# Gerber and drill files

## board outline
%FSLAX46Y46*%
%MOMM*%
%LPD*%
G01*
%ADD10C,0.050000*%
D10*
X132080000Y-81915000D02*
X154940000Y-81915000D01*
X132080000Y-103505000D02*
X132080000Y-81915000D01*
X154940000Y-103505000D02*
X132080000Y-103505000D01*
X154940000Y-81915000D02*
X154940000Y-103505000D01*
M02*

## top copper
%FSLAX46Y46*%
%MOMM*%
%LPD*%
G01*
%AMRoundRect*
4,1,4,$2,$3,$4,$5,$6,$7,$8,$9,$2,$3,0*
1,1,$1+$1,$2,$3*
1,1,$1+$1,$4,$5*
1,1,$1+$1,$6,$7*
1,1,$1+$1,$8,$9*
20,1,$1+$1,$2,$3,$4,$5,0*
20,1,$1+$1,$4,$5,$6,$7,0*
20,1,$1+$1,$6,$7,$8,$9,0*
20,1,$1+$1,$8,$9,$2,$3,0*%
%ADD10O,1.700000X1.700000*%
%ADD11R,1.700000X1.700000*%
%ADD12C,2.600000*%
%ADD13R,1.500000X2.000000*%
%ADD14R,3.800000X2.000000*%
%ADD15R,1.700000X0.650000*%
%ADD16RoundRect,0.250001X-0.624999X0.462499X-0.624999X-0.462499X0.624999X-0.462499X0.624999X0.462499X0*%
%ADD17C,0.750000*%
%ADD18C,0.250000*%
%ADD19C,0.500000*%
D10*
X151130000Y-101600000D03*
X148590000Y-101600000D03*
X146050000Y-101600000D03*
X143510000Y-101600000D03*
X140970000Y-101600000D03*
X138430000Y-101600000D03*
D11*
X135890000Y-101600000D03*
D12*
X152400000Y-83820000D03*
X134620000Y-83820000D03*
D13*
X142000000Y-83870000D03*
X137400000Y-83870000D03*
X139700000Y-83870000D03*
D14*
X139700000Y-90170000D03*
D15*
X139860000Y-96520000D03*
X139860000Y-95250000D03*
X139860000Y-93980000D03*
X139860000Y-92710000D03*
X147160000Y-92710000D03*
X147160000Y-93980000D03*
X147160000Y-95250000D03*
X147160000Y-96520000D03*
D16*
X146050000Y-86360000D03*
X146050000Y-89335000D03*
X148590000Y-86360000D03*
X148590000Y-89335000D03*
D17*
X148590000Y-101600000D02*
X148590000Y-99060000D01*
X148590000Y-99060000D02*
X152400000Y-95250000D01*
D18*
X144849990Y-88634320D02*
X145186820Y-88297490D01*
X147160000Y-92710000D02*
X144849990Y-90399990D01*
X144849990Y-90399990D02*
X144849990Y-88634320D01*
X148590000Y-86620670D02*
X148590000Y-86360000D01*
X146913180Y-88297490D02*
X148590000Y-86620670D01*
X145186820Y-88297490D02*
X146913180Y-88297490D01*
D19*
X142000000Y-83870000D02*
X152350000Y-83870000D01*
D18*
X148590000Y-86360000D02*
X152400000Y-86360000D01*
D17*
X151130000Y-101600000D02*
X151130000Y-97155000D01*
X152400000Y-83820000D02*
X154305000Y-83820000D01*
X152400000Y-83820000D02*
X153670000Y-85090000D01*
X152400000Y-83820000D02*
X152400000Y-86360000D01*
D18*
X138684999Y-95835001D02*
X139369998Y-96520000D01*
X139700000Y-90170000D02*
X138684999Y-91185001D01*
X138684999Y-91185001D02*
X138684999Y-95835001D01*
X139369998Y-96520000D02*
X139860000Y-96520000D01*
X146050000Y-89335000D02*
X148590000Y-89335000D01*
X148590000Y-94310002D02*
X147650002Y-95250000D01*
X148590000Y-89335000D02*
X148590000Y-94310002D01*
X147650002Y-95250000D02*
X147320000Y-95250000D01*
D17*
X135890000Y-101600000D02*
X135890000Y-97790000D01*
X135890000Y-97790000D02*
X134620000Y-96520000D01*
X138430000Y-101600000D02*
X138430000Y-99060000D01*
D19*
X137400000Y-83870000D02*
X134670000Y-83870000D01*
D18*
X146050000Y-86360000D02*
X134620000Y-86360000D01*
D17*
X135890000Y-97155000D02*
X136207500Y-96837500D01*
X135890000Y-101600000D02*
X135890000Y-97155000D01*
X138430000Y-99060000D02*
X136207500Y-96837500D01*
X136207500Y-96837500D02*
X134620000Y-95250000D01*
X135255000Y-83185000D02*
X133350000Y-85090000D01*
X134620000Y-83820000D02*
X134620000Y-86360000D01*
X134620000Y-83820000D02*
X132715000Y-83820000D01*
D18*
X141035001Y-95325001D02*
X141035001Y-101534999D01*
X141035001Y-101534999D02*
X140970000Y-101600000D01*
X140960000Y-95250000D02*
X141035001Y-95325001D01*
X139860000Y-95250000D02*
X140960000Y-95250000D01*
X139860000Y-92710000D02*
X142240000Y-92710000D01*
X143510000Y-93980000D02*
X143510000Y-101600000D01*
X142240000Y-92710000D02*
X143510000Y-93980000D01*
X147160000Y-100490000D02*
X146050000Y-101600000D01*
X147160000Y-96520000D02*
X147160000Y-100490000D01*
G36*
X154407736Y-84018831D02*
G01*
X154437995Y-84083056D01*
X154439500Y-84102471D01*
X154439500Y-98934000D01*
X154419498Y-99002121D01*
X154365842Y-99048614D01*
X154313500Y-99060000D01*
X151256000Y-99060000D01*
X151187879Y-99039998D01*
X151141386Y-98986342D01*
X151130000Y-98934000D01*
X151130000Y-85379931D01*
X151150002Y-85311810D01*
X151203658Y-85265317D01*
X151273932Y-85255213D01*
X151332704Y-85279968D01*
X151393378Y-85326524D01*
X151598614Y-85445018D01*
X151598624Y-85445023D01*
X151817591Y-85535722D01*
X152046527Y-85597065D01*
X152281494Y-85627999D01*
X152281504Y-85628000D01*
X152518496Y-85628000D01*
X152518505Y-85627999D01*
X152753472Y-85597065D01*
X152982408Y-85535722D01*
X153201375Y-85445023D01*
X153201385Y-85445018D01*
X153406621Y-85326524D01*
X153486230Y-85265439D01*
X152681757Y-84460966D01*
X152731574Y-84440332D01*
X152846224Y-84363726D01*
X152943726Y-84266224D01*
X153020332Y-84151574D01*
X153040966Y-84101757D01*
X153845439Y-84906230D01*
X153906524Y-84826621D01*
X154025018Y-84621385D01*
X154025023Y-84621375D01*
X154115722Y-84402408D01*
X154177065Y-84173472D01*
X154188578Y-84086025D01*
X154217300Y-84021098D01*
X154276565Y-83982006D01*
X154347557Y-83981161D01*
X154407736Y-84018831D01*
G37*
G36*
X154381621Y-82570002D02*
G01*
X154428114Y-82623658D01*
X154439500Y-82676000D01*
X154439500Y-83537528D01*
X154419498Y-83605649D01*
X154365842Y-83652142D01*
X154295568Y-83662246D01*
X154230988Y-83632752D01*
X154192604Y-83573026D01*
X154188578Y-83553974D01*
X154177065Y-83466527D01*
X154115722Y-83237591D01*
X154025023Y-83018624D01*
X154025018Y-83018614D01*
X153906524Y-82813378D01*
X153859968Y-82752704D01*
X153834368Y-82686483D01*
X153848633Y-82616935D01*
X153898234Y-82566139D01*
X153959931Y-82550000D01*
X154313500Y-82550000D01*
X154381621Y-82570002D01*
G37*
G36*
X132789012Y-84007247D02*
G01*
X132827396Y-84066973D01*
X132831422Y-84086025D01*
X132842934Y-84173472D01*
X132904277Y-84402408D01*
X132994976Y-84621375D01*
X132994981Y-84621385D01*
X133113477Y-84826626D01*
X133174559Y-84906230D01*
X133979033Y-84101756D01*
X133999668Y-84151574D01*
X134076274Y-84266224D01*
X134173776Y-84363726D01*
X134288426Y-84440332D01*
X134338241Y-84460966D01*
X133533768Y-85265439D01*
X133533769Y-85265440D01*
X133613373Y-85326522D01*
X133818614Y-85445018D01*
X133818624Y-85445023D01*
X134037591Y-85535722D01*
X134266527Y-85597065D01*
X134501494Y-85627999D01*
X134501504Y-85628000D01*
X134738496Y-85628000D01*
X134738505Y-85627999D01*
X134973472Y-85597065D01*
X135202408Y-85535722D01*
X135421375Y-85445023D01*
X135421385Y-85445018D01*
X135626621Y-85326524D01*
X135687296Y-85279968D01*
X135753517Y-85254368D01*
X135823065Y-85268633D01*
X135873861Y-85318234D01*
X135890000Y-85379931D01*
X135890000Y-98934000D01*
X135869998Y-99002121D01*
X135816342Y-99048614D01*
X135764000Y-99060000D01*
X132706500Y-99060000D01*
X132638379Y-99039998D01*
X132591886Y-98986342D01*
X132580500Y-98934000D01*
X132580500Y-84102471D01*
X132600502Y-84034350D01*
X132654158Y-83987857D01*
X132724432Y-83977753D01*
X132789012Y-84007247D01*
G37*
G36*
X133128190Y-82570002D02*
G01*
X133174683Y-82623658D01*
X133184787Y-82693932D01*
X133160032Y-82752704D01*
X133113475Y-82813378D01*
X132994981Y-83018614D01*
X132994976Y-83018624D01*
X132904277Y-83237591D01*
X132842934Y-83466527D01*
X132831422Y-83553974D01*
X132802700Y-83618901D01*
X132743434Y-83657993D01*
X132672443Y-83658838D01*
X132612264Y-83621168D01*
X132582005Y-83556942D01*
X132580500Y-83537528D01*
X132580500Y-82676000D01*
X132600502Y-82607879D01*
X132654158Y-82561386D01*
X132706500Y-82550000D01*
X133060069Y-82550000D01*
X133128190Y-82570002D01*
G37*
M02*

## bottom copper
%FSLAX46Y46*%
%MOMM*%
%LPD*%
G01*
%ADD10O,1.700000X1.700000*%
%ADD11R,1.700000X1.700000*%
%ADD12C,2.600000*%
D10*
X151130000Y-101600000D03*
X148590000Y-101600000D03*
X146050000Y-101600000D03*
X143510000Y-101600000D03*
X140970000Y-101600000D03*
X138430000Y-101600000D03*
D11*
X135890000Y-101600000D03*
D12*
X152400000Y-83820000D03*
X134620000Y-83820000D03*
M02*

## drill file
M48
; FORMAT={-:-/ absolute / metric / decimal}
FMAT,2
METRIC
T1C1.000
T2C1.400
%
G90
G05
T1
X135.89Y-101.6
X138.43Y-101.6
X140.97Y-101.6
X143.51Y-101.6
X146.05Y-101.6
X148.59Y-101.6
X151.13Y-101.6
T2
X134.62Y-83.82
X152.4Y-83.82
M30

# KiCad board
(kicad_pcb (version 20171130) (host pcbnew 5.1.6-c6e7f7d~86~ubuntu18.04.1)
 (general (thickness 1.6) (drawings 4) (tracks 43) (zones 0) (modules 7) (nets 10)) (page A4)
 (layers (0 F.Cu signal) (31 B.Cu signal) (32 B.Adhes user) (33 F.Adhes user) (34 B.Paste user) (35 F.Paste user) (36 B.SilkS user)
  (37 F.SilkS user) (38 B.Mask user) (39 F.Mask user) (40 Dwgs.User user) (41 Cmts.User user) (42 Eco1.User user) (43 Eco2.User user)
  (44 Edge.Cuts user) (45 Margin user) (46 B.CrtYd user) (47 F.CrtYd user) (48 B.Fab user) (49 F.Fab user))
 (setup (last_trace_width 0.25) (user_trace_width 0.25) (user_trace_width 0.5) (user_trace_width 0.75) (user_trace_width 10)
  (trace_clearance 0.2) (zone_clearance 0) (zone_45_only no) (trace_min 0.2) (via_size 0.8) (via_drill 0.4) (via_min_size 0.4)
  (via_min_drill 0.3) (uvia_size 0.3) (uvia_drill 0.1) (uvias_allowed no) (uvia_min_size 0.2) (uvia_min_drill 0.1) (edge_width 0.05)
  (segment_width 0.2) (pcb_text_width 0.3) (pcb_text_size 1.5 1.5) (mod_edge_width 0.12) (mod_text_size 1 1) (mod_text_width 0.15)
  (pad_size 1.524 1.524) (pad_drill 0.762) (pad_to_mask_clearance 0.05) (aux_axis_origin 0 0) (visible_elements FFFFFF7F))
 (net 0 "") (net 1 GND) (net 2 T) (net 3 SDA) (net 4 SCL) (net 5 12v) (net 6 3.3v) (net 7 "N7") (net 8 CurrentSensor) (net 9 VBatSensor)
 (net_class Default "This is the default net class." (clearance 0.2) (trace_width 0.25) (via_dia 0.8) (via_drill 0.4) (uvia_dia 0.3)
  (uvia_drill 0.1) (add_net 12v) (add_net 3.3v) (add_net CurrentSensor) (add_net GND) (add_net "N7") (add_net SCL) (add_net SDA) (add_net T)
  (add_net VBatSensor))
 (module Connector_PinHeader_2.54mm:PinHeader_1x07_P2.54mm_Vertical (layer F.Cu) (at 135.89 101.6 90)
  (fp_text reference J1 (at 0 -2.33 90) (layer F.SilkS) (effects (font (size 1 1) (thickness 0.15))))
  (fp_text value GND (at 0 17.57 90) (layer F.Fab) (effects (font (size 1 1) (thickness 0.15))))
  (pad 7 thru_hole oval (at 0 15.24 90) (size 1.7 1.7) (drill 1) (layers *.Cu *.Mask) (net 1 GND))
  (pad 6 thru_hole oval (at 0 12.7 90) (size 1.7 1.7) (drill 1) (layers *.Cu *.Mask) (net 1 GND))
  (pad 5 thru_hole oval (at 0 10.16 90) (size 1.7 1.7) (drill 1) (layers *.Cu *.Mask) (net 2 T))
  (pad 4 thru_hole oval (at 0 7.62 90) (size 1.7 1.7) (drill 1) (layers *.Cu *.Mask) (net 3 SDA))
  (pad 3 thru_hole oval (at 0 5.08 90) (size 1.7 1.7) (drill 1) (layers *.Cu *.Mask) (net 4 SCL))
  (pad 2 thru_hole oval (at 0 2.54 90) (size 1.7 1.7) (drill 1) (layers *.Cu *.Mask) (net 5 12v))
  (pad 1 thru_hole rect (at 0 0 90) (size 1.7 1.7) (drill 1) (layers *.Cu *.Mask) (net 5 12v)))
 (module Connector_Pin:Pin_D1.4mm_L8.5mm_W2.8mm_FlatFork (layer F.Cu) (at 152.4 83.82)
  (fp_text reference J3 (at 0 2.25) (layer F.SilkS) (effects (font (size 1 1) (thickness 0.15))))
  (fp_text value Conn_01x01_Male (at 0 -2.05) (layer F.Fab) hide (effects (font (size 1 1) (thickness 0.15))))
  (pad 1 thru_hole circle (at 0 0) (size 2.6 2.6) (drill 1.4) (layers *.Cu *.Mask) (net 1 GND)))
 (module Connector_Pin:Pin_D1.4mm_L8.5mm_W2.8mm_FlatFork (layer F.Cu) (at 134.62 83.82)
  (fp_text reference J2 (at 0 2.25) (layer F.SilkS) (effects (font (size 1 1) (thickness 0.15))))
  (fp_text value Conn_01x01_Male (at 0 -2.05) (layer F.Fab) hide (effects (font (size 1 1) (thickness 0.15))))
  (pad 1 thru_hole circle (at 0 0) (size 2.6 2.6) (drill 1.4) (layers *.Cu *.Mask) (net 5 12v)))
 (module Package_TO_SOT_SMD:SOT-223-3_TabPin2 (layer F.Cu) (at 139.7 87.02 270)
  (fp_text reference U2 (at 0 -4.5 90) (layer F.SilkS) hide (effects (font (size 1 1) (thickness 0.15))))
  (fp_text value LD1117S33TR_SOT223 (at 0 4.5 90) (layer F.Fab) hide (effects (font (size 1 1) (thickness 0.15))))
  (pad 1 smd rect (at -3.15 -2.3 270) (size 2 1.5) (layers F.Cu F.Paste F.Mask) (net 1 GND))
  (pad 3 smd rect (at -3.15 2.3 270) (size 2 1.5) (layers F.Cu F.Paste F.Mask) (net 5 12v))
  (pad 2 smd rect (at -3.15 0 270) (size 2 1.5) (layers F.Cu F.Paste F.Mask) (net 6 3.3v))
  (pad 2 smd rect (at 3.15 0 270) (size 2 3.8) (layers F.Cu F.Paste F.Mask) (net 6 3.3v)))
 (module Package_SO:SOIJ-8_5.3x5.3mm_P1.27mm (layer F.Cu) (at 143.51 94.615 180)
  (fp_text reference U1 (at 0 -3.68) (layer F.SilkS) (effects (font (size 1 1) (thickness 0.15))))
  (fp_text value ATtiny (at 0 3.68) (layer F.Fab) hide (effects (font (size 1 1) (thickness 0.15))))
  (pad 8 smd rect (at 3.65 -1.905 180) (size 1.7 0.65) (layers F.Cu F.Paste F.Mask) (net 6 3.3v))
  (pad 7 smd rect (at 3.65 -0.635 180) (size 1.7 0.65) (layers F.Cu F.Paste F.Mask) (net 4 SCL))
  (pad 6 smd rect (at 3.65 0.635 180) (size 1.7 0.65) (layers F.Cu F.Paste F.Mask) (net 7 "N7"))
  (pad 5 smd rect (at 3.65 1.905 180) (size 1.7 0.65) (layers F.Cu F.Paste F.Mask) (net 3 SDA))
  (pad 4 smd rect (at -3.65 1.905 180) (size 1.7 0.65) (layers F.Cu F.Paste F.Mask) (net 1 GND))
  (pad 3 smd rect (at -3.65 0.635 180) (size 1.7 0.65) (layers F.Cu F.Paste F.Mask) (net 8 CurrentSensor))
  (pad 2 smd rect (at -3.65 -0.635 180) (size 1.7 0.65) (layers F.Cu F.Paste F.Mask) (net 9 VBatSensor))
  (pad 1 smd rect (at -3.65 -1.905 180) (size 1.7 0.65) (layers F.Cu F.Paste F.Mask) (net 2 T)))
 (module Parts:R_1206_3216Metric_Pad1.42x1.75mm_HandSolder (layer F.Cu) (at 146.05 87.8475 270)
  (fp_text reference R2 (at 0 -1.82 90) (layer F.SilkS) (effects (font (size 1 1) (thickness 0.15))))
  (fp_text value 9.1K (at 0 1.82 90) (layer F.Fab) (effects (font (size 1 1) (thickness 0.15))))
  (pad 1 smd roundrect (at -1.4875 0 270) (size 1.425 1.75) (layers F.Cu F.Paste F.Mask) (roundrect_rratio 0.175439) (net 5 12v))
  (pad 2 smd roundrect (at 1.4875 0 270) (size 1.425 1.75) (layers F.Cu F.Paste F.Mask) (roundrect_rratio 0.175439) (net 9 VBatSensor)))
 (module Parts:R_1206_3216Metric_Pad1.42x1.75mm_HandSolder (layer F.Cu) (at 148.59 87.8475 270)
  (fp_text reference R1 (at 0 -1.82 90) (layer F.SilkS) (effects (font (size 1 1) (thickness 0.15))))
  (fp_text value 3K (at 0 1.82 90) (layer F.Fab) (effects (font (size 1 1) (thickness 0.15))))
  (pad 1 smd roundrect (at -1.4875 0 270) (size 1.425 1.75) (layers F.Cu F.Paste F.Mask) (roundrect_rratio 0.175439) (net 1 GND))
  (pad 2 smd roundrect (at 1.4875 0 270) (size 1.425 1.75) (layers F.Cu F.Paste F.Mask) (roundrect_rratio 0.175439) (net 9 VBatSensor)))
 (gr_line (start 132.08 81.915) (end 154.94 81.915) (layer Edge.Cuts) (width 0.05))
 (gr_line (start 132.08 103.505) (end 132.08 81.915) (layer Edge.Cuts) (width 0.05))
 (gr_line (start 154.94 103.505) (end 132.08 103.505) (layer Edge.Cuts) (width 0.05))
 (gr_line (start 154.94 81.915) (end 154.94 103.505) (layer Edge.Cuts) (width 0.05))
 (segment (start 148.59 101.6) (end 148.59 99.06) (width 0.75) (layer F.Cu) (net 1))
 (segment (start 148.59 99.06) (end 152.4 95.25) (width 0.75) (layer F.Cu) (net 1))
 (segment (start 144.84999 88.63432) (end 145.18682 88.29749) (width 0.25) (layer F.Cu) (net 1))
 (segment (start 147.16 92.71) (end 144.84999 90.39999) (width 0.25) (layer F.Cu) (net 1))
 (segment (start 144.84999 90.39999) (end 144.84999 88.63432) (width 0.25) (layer F.Cu) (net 1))
 (segment (start 148.59 86.62067) (end 148.59 86.36) (width 0.25) (layer F.Cu) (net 1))
 (segment (start 146.91318 88.29749) (end 148.59 86.62067) (width 0.25) (layer F.Cu) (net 1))
 (segment (start 145.18682 88.29749) (end 146.91318 88.29749) (width 0.25) (layer F.Cu) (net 1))
 (segment (start 142 83.87) (end 152.35 83.87) (width 0.5) (layer F.Cu) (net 1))
 (segment (start 148.59 86.36) (end 152.4 86.36) (width 0.25) (layer F.Cu) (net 1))
 (segment (start 151.13 101.6) (end 151.13 97.155) (width 0.75) (layer F.Cu) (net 1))
 (segment (start 152.4 83.82) (end 154.305 83.82) (width 0.75) (layer F.Cu) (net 1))
 (segment (start 152.4 83.82) (end 153.67 85.09) (width 0.75) (layer F.Cu) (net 1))
 (segment (start 152.4 83.82) (end 152.4 86.36) (width 0.75) (layer F.Cu) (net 1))
 (segment (start 138.684999 95.835001) (end 139.369998 96.52) (width 0.25) (layer F.Cu) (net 6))
 (segment (start 139.7 90.17) (end 138.684999 91.185001) (width 0.25) (layer F.Cu) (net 6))
 (segment (start 138.684999 91.185001) (end 138.684999 95.835001) (width 0.25) (layer F.Cu) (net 6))
 (segment (start 139.369998 96.52) (end 139.86 96.52) (width 0.25) (layer F.Cu) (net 6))
 (segment (start 146.05 89.335) (end 148.59 89.335) (width 0.25) (layer F.Cu) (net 9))
 (segment (start 148.59 94.310002) (end 147.650002 95.25) (width 0.25) (layer F.Cu) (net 9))
 (segment (start 148.59 89.335) (end 148.59 94.310002) (width 0.25) (layer F.Cu) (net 9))
 (segment (start 147.650002 95.25) (end 147.32 95.25) (width 0.25) (layer F.Cu) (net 9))
 (segment (start 135.89 101.6) (end 135.89 97.79) (width 0.75) (layer F.Cu) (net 5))
 (segment (start 135.89 97.79) (end 134.62 96.52) (width 0.75) (layer F.Cu) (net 5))
 (segment (start 138.43 101.6) (end 138.43 99.06) (width 0.75) (layer F.Cu) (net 5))
 (segment (start 137.4 83.87) (end 134.67 83.87) (width 0.5) (layer F.Cu) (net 5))
 (segment (start 146.05 86.36) (end 134.62 86.36) (width 0.25) (layer F.Cu) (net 5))
 (segment (start 135.89 97.155) (end 136.2075 96.8375) (width 0.75) (layer F.Cu) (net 5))
 (segment (start 135.89 101.6) (end 135.89 97.155) (width 0.75) (layer F.Cu) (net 5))
 (segment (start 138.43 99.06) (end 136.2075 96.8375) (width 0.75) (layer F.Cu) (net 5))
 (segment (start 136.2075 96.8375) (end 134.62 95.25) (width 0.75) (layer F.Cu) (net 5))
 (segment (start 135.255 83.185) (end 133.35 85.09) (width 0.75) (layer F.Cu) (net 5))
 (segment (start 134.62 83.82) (end 134.62 86.36) (width 0.75) (layer F.Cu) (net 5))
 (segment (start 134.62 83.82) (end 132.715 83.82) (width 0.75) (layer F.Cu) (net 5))
 (segment (start 141.035001 95.325001) (end 141.035001 101.534999) (width 0.25) (layer F.Cu) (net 4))
 (segment (start 141.035001 101.534999) (end 140.97 101.6) (width 0.25) (layer F.Cu) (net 4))
 (segment (start 140.96 95.25) (end 141.035001 95.325001) (width 0.25) (layer F.Cu) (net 4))
 (segment (start 139.86 95.25) (end 140.96 95.25) (width 0.25) (layer F.Cu) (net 4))
 (segment (start 139.86 92.71) (end 142.24 92.71) (width 0.25) (layer F.Cu) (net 3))
 (segment (start 143.51 93.98) (end 143.51 101.6) (width 0.25) (layer F.Cu) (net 3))
 (segment (start 142.24 92.71) (end 143.51 93.98) (width 0.25) (layer F.Cu) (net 3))
 (segment (start 147.16 100.49) (end 146.05 101.6) (width 0.25) (layer F.Cu) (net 2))
 (segment (start 147.16 96.52) (end 147.16 100.49) (width 0.25) (layer F.Cu) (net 2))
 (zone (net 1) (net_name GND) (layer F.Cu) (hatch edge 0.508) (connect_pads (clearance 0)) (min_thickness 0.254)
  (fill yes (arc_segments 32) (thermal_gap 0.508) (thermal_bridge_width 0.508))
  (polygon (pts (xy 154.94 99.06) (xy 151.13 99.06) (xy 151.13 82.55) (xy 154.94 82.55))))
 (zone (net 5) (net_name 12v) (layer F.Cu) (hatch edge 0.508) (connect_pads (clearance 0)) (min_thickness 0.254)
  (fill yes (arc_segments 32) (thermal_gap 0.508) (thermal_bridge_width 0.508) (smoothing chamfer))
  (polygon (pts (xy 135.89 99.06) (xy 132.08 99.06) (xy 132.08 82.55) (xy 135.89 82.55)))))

